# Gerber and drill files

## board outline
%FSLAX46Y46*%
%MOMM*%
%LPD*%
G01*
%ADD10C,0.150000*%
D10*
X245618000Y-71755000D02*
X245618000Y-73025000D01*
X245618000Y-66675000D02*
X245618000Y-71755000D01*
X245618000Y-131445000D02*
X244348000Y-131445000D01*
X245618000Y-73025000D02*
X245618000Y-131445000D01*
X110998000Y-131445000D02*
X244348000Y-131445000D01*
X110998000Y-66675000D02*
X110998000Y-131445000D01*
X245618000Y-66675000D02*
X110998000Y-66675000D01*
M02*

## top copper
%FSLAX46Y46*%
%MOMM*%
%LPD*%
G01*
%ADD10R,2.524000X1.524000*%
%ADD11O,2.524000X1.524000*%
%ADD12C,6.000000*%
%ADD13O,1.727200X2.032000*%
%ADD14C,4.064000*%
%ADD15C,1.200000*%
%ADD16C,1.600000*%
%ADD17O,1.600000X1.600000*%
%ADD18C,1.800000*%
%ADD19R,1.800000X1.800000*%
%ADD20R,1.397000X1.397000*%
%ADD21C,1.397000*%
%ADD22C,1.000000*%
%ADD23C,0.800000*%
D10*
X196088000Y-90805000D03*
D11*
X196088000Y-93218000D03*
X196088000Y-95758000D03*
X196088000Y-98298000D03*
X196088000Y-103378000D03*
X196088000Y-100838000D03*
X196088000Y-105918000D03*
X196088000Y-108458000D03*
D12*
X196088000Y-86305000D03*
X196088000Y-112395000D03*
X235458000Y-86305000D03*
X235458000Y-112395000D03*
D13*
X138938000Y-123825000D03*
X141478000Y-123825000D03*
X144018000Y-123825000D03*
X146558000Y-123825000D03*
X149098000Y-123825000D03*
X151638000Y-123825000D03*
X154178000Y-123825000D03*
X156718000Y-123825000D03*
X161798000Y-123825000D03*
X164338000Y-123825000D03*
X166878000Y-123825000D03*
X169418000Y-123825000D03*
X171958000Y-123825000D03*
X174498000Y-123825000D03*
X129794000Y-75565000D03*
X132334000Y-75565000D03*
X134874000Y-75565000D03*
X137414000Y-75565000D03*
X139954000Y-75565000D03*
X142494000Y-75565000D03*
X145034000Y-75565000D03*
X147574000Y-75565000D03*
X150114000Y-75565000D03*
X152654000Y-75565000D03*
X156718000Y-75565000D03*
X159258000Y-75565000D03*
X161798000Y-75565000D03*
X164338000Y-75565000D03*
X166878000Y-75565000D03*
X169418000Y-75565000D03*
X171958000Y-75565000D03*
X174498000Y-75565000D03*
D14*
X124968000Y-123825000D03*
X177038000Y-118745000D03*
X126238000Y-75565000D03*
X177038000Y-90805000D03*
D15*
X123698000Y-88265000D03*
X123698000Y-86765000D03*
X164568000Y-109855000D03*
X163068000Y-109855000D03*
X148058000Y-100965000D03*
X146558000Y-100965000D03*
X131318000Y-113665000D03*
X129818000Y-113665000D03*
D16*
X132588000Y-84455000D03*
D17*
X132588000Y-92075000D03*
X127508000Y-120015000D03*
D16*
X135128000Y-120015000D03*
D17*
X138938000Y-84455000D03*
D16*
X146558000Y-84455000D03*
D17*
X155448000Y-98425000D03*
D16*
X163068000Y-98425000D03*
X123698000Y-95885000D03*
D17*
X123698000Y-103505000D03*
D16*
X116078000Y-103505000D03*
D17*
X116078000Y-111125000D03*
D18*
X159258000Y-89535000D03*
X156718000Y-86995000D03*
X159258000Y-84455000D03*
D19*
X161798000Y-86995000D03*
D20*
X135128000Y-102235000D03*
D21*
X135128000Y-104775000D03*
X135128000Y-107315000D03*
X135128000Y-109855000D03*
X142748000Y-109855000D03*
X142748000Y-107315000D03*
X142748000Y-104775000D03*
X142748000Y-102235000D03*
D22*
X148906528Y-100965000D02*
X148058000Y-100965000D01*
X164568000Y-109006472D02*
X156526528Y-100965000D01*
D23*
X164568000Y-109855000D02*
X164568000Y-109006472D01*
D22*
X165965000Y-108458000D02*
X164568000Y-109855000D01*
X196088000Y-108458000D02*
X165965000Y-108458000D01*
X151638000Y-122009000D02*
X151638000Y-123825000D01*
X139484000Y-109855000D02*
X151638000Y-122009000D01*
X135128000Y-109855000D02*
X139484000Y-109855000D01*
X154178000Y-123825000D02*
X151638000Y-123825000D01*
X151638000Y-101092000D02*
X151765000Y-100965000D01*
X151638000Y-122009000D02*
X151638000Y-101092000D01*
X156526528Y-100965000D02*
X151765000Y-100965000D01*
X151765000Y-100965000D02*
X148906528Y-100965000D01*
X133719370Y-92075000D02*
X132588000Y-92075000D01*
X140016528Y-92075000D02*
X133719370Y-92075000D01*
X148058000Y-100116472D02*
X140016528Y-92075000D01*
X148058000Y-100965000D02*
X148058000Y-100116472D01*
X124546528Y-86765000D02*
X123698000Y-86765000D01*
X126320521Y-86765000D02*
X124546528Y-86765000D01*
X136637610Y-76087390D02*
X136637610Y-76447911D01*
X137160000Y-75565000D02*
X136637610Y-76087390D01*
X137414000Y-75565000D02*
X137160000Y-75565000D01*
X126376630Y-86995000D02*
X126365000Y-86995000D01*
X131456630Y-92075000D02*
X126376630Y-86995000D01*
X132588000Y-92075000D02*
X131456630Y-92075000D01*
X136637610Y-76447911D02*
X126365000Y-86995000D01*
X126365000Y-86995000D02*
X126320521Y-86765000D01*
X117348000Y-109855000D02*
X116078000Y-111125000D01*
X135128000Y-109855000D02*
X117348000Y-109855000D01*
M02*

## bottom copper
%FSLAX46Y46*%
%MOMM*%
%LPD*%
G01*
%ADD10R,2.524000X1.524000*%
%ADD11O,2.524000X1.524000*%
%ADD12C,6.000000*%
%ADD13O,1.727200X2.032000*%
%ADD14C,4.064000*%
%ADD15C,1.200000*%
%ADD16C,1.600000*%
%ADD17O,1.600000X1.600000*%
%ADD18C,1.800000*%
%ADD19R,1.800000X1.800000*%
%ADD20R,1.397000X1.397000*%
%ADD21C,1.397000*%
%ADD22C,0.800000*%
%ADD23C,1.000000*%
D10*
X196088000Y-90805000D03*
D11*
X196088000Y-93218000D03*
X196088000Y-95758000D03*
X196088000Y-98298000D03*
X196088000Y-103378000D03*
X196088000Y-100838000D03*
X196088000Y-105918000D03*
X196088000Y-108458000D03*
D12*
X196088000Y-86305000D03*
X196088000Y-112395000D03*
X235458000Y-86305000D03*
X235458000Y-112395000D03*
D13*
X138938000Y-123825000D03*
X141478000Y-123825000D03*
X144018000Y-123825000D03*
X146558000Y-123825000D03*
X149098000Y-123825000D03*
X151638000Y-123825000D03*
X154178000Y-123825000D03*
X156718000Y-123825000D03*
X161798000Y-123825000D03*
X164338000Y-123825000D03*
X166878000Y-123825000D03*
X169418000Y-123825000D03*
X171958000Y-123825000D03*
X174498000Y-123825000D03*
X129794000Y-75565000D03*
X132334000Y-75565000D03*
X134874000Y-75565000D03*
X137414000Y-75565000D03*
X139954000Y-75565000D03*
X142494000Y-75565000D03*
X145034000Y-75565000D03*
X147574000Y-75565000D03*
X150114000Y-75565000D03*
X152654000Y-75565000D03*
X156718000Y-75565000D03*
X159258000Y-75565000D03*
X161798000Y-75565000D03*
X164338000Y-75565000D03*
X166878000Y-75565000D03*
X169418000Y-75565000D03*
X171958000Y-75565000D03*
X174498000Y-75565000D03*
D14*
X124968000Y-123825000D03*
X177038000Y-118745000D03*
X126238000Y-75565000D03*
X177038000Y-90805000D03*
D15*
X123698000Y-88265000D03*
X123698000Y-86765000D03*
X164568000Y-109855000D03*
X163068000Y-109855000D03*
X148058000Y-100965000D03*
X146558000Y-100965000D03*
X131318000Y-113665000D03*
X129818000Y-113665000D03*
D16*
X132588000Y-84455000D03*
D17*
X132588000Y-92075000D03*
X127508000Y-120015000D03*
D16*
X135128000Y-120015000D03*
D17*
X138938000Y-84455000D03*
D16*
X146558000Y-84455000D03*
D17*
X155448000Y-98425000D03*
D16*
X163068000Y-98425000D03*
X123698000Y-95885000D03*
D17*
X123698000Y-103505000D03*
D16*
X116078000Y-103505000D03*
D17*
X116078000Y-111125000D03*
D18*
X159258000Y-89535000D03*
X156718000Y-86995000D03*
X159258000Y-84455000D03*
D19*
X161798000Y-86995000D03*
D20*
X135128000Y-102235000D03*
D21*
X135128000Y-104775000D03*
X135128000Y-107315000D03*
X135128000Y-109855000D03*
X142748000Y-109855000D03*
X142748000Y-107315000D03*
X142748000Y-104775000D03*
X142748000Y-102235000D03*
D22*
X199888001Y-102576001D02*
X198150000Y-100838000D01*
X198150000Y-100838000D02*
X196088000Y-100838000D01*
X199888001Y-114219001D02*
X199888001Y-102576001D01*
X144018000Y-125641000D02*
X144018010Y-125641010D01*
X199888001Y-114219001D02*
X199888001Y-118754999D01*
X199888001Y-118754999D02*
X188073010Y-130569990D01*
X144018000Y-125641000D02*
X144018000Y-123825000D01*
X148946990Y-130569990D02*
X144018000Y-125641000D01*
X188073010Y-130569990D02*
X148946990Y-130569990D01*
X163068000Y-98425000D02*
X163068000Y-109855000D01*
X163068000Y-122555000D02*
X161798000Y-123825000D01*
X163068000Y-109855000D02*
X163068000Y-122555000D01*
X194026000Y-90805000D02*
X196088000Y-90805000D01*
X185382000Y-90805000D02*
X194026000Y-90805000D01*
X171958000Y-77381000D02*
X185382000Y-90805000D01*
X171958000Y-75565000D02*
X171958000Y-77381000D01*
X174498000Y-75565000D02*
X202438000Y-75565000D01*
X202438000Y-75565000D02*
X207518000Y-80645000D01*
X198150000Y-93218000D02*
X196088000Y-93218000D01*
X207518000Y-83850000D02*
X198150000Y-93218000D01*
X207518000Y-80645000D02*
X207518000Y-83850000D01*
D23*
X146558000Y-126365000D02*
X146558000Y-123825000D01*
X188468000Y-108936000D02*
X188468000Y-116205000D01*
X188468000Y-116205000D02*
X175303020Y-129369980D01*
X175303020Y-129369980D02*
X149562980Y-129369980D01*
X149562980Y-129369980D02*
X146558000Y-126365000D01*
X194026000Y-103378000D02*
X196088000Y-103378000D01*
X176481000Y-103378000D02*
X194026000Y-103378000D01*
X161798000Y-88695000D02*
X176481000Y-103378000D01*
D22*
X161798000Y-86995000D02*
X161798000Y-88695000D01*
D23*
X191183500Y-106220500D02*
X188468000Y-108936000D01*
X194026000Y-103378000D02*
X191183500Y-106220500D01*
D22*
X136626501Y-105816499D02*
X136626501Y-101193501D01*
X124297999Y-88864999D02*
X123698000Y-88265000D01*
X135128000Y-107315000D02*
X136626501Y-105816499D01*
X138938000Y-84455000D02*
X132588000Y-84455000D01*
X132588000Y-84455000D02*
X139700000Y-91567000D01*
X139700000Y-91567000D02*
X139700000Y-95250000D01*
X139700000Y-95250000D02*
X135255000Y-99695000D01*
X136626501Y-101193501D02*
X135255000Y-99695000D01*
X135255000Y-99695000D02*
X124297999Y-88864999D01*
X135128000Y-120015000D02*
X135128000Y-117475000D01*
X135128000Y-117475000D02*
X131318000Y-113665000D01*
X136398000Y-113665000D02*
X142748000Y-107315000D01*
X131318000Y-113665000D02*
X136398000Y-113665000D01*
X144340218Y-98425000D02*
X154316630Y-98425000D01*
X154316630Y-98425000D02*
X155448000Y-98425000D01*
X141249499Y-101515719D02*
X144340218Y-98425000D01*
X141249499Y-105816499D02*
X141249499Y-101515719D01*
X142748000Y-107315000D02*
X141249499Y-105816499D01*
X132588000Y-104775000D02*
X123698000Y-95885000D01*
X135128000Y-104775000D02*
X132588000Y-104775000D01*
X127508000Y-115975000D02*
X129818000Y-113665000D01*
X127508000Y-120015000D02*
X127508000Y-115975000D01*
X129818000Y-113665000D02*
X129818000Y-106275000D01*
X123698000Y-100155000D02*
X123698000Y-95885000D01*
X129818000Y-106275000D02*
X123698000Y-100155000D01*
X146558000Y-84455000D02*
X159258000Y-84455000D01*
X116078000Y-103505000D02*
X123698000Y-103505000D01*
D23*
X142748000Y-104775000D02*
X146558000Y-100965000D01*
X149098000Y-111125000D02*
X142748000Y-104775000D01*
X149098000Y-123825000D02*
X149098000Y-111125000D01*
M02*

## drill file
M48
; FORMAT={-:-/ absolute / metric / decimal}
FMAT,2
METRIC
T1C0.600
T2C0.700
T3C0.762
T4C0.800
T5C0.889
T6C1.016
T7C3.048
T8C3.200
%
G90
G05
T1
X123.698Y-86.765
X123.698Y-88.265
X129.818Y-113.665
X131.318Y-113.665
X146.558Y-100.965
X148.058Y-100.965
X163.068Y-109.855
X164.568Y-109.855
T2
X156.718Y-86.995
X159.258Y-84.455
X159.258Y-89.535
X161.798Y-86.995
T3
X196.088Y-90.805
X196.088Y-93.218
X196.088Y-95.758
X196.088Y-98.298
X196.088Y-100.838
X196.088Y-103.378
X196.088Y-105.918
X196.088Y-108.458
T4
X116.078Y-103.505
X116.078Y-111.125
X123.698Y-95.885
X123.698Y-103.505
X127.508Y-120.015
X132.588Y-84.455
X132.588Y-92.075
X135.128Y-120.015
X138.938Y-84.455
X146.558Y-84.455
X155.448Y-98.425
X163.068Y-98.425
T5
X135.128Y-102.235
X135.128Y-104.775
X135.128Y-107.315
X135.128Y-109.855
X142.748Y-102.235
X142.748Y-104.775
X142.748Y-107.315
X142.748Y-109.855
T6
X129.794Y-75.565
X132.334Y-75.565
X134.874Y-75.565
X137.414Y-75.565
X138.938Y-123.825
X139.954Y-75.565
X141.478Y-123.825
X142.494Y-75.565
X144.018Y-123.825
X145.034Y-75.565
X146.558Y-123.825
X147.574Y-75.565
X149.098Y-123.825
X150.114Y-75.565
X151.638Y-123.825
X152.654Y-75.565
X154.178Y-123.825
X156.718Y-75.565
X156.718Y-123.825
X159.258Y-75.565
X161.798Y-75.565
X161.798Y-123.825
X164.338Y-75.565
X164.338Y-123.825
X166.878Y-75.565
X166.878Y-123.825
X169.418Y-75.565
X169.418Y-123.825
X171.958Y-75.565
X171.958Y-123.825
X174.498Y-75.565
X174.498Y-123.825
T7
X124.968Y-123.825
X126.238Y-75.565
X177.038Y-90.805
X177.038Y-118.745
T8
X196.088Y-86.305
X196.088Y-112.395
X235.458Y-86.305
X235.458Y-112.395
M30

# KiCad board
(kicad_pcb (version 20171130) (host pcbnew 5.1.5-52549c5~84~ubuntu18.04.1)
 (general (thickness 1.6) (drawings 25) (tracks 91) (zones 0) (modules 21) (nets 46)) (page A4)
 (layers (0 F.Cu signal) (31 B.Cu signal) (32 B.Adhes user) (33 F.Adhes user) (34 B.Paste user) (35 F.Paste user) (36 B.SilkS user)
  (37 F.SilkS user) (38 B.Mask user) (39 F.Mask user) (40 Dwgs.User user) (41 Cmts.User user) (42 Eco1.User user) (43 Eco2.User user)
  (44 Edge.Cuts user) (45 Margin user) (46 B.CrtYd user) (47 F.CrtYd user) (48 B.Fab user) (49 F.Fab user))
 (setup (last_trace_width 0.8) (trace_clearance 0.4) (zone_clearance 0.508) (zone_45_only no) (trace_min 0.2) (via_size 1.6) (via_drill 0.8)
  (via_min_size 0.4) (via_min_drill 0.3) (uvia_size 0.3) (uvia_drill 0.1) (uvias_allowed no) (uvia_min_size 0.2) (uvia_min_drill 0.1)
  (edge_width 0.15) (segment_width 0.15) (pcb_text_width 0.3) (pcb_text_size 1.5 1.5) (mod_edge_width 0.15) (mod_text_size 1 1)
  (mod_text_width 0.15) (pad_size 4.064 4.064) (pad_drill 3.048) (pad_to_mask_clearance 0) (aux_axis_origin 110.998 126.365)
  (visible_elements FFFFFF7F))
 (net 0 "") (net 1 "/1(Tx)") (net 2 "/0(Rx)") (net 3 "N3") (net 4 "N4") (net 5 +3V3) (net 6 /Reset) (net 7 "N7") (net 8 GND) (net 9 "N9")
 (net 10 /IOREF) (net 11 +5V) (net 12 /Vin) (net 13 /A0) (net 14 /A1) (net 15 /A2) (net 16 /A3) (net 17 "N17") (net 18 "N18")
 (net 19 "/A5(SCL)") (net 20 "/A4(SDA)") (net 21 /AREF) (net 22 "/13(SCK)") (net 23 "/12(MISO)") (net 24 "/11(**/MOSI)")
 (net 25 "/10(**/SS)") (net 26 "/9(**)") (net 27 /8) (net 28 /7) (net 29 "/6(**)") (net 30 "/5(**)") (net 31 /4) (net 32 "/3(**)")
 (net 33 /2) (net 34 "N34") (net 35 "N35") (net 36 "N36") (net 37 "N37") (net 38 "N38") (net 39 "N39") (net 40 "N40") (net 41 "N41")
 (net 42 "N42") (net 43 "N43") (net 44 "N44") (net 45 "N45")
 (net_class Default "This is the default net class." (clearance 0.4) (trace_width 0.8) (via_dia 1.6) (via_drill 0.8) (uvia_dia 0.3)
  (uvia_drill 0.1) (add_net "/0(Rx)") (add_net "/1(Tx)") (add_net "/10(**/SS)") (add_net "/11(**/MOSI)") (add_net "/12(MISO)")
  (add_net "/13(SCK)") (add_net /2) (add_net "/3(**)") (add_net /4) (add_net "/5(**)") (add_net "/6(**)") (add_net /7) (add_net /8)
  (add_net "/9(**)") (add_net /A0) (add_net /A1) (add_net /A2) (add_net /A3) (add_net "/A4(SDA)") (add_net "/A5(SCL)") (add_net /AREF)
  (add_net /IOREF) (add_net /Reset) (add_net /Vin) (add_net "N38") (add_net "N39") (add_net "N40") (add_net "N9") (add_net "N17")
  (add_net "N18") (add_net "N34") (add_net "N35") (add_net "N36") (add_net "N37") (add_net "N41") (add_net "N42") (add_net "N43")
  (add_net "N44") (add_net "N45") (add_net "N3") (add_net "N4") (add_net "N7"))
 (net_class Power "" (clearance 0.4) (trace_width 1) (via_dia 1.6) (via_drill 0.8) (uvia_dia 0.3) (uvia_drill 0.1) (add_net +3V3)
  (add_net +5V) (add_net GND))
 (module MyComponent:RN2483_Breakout (layer F.Cu) (at 196.088 90.805 270)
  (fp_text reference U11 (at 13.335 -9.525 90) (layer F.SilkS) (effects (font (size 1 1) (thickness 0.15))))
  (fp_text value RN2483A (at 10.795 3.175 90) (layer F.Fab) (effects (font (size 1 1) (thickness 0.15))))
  (pad 1 thru_hole rect (at 0 0 270) (size 1.524 2.524) (drill 0.762) (layers *.Cu *.Mask) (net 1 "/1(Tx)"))
  (pad 2 thru_hole oval (at 2.413 0 270) (size 1.524 2.524) (drill 0.762) (layers *.Cu *.Mask) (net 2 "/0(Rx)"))
  (pad 3 thru_hole oval (at 4.953 0 270) (size 1.524 2.524) (drill 0.762) (layers *.Cu *.Mask) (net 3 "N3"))
  (pad 4 thru_hole oval (at 7.493 0 270) (size 1.524 2.524) (drill 0.762) (layers *.Cu *.Mask) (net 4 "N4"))
  (pad 6 thru_hole oval (at 12.573 0 270) (size 1.524 2.524) (drill 0.762) (layers *.Cu *.Mask) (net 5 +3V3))
  (pad 5 thru_hole oval (at 10.033 0 270) (size 1.524 2.524) (drill 0.762) (layers *.Cu *.Mask) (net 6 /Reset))
  (pad 7 thru_hole oval (at 15.113 0 270) (size 1.524 2.524) (drill 0.762) (layers *.Cu *.Mask) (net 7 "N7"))
  (pad 8 thru_hole oval (at 17.653 0 270) (size 1.524 2.524) (drill 0.762) (layers *.Cu *.Mask) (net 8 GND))
  (pad "" np_thru_hole circle (at -4.5 0 270) (size 6 6) (drill 3.2) (layers *.Cu *.Mask))
  (pad "" np_thru_hole circle (at 21.59 0 270) (size 6 6) (drill 3.2) (layers *.Cu *.Mask))
  (pad "" np_thru_hole circle (at -4.5 -39.37 270) (size 6 6) (drill 3.2) (layers *.Cu *.Mask))
  (pad "" np_thru_hole circle (at 21.59 -39.37 270) (size 6 6) (drill 3.2) (layers *.Cu *.Mask)))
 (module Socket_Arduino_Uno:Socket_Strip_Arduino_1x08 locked (layer F.Cu) (at 138.938 123.825)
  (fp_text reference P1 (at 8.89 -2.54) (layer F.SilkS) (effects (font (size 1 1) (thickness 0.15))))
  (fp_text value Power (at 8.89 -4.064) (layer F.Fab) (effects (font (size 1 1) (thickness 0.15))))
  (pad 1 thru_hole oval (at 0 0) (size 1.7272 2.032) (drill 1.016) (layers *.Cu *.Mask F.SilkS) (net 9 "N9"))
  (pad 2 thru_hole oval (at 2.54 0) (size 1.7272 2.032) (drill 1.016) (layers *.Cu *.Mask F.SilkS) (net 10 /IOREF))
  (pad 3 thru_hole oval (at 5.08 0) (size 1.7272 2.032) (drill 1.016) (layers *.Cu *.Mask F.SilkS) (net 6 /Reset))
  (pad 4 thru_hole oval (at 7.62 0) (size 1.7272 2.032) (drill 1.016) (layers *.Cu *.Mask F.SilkS) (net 5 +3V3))
  (pad 5 thru_hole oval (at 10.16 0) (size 1.7272 2.032) (drill 1.016) (layers *.Cu *.Mask F.SilkS) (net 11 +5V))
  (pad 6 thru_hole oval (at 12.7 0) (size 1.7272 2.032) (drill 1.016) (layers *.Cu *.Mask F.SilkS) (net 8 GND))
  (pad 7 thru_hole oval (at 15.24 0) (size 1.7272 2.032) (drill 1.016) (layers *.Cu *.Mask F.SilkS) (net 8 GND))
  (pad 8 thru_hole oval (at 17.78 0) (size 1.7272 2.032) (drill 1.016) (layers *.Cu *.Mask F.SilkS) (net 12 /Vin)))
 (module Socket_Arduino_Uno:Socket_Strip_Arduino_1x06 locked (layer F.Cu) (at 161.798 123.825)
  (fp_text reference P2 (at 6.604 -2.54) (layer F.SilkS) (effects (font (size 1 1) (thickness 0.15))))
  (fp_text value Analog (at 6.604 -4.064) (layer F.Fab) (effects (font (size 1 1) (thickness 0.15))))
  (pad 1 thru_hole oval (at 0 0) (size 1.7272 2.032) (drill 1.016) (layers *.Cu *.Mask F.SilkS) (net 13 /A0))
  (pad 2 thru_hole oval (at 2.54 0) (size 1.7272 2.032) (drill 1.016) (layers *.Cu *.Mask F.SilkS) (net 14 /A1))
  (pad 3 thru_hole oval (at 5.08 0) (size 1.7272 2.032) (drill 1.016) (layers *.Cu *.Mask F.SilkS) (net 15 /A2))
  (pad 4 thru_hole oval (at 7.62 0) (size 1.7272 2.032) (drill 1.016) (layers *.Cu *.Mask F.SilkS) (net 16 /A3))
  (pad 5 thru_hole oval (at 10.16 0) (size 1.7272 2.032) (drill 1.016) (layers *.Cu *.Mask F.SilkS) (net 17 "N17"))
  (pad 6 thru_hole oval (at 12.7 0) (size 1.7272 2.032) (drill 1.016) (layers *.Cu *.Mask F.SilkS) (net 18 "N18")))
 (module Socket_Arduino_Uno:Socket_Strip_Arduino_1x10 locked (layer F.Cu) (at 129.794 75.565)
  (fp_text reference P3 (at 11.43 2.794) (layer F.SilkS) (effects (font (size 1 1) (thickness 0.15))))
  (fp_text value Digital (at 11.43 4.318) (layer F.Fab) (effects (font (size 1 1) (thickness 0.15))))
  (pad 1 thru_hole oval (at 0 0) (size 1.7272 2.032) (drill 1.016) (layers *.Cu *.Mask F.SilkS) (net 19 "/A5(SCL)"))
  (pad 2 thru_hole oval (at 2.54 0) (size 1.7272 2.032) (drill 1.016) (layers *.Cu *.Mask F.SilkS) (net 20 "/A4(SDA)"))
  (pad 3 thru_hole oval (at 5.08 0) (size 1.7272 2.032) (drill 1.016) (layers *.Cu *.Mask F.SilkS) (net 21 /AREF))
  (pad 4 thru_hole oval (at 7.62 0) (size 1.7272 2.032) (drill 1.016) (layers *.Cu *.Mask F.SilkS) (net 8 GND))
  (pad 5 thru_hole oval (at 10.16 0) (size 1.7272 2.032) (drill 1.016) (layers *.Cu *.Mask F.SilkS) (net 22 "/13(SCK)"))
  (pad 6 thru_hole oval (at 12.7 0) (size 1.7272 2.032) (drill 1.016) (layers *.Cu *.Mask F.SilkS) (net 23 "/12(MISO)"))
  (pad 7 thru_hole oval (at 15.24 0) (size 1.7272 2.032) (drill 1.016) (layers *.Cu *.Mask F.SilkS) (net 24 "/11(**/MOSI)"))
  (pad 8 thru_hole oval (at 17.78 0) (size 1.7272 2.032) (drill 1.016) (layers *.Cu *.Mask F.SilkS) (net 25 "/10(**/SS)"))
  (pad 9 thru_hole oval (at 20.32 0) (size 1.7272 2.032) (drill 1.016) (layers *.Cu *.Mask F.SilkS) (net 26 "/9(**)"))
  (pad 10 thru_hole oval (at 22.86 0) (size 1.7272 2.032) (drill 1.016) (layers *.Cu *.Mask F.SilkS) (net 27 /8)))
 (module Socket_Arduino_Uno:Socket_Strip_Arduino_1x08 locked (layer F.Cu) (at 156.718 75.565)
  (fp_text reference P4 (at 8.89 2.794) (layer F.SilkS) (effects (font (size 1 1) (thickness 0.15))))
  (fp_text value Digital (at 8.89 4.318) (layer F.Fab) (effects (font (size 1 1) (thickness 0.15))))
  (pad 1 thru_hole oval (at 0 0) (size 1.7272 2.032) (drill 1.016) (layers *.Cu *.Mask F.SilkS) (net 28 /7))
  (pad 2 thru_hole oval (at 2.54 0) (size 1.7272 2.032) (drill 1.016) (layers *.Cu *.Mask F.SilkS) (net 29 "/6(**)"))
  (pad 3 thru_hole oval (at 5.08 0) (size 1.7272 2.032) (drill 1.016) (layers *.Cu *.Mask F.SilkS) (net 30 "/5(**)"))
  (pad 4 thru_hole oval (at 7.62 0) (size 1.7272 2.032) (drill 1.016) (layers *.Cu *.Mask F.SilkS) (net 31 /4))
  (pad 5 thru_hole oval (at 10.16 0) (size 1.7272 2.032) (drill 1.016) (layers *.Cu *.Mask F.SilkS) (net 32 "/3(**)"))
  (pad 6 thru_hole oval (at 12.7 0) (size 1.7272 2.032) (drill 1.016) (layers *.Cu *.Mask F.SilkS) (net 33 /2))
  (pad 7 thru_hole oval (at 15.24 0) (size 1.7272 2.032) (drill 1.016) (layers *.Cu *.Mask F.SilkS) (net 1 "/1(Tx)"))
  (pad 8 thru_hole oval (at 17.78 0) (size 1.7272 2.032) (drill 1.016) (layers *.Cu *.Mask F.SilkS) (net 2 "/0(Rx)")))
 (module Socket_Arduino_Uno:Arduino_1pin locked (layer F.Cu) (at 124.968 123.825)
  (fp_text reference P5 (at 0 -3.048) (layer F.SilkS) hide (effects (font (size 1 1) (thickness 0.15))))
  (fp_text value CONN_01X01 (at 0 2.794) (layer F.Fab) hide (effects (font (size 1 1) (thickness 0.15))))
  (pad 1 thru_hole circle (at 0 0) (size 4.064 4.064) (drill 3.048) (layers *.Cu *.Mask F.SilkS) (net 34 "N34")))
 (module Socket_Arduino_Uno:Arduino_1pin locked (layer F.Cu) (at 177.038 118.745)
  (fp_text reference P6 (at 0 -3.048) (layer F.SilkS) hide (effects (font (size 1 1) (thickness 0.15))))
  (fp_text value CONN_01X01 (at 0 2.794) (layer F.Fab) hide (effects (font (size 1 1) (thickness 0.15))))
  (pad 1 thru_hole circle (at 0 0) (size 4.064 4.064) (drill 3.048) (layers *.Cu *.Mask F.SilkS) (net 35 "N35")))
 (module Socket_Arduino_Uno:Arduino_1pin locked (layer F.Cu) (at 126.238 75.565)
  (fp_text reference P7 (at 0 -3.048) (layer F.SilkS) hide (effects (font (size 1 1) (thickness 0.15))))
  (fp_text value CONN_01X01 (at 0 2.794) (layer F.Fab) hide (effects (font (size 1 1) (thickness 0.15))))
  (pad 1 thru_hole circle (at 0 0) (size 4.064 4.064) (drill 3.048) (layers *.Cu *.Mask F.SilkS) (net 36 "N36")))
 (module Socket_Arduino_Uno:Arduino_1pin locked (layer F.Cu) (at 177.038 90.805)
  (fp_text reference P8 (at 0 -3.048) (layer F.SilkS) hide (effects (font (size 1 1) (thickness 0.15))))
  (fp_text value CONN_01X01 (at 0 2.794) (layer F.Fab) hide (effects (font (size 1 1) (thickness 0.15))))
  (pad 1 thru_hole circle (at 0 0) (size 4.064 4.064) (drill 3.048) (layers *.Cu *.Mask F.SilkS) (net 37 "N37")))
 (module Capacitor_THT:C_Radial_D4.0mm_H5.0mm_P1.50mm (layer F.Cu) (at 123.698 88.265 90)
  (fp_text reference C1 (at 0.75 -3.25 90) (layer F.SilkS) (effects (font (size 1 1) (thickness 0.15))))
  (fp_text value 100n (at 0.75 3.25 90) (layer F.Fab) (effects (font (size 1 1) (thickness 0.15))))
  (pad 1 thru_hole circle (at 0 0 90) (size 1.2 1.2) (drill 0.6) (layers *.Cu *.Mask) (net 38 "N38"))
  (pad 2 thru_hole circle (at 1.5 0 90) (size 1.2 1.2) (drill 0.6) (layers *.Cu *.Mask) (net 8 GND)))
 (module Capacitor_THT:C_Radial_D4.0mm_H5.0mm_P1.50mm (layer F.Cu) (at 163.068 109.855)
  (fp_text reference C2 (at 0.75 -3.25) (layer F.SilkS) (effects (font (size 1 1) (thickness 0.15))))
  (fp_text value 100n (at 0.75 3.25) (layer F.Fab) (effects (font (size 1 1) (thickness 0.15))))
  (pad 2 thru_hole circle (at 1.5 0) (size 1.2 1.2) (drill 0.6) (layers *.Cu *.Mask) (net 8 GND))
  (pad 1 thru_hole circle (at 0 0) (size 1.2 1.2) (drill 0.6) (layers *.Cu *.Mask) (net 13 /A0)))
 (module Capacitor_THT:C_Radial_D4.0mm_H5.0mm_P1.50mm (layer F.Cu) (at 146.558 100.965)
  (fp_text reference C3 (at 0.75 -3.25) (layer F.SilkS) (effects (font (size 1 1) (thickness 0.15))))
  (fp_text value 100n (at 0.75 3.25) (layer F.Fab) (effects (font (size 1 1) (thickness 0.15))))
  (pad 2 thru_hole circle (at 1.5 0) (size 1.2 1.2) (drill 0.6) (layers *.Cu *.Mask) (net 8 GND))
  (pad 1 thru_hole circle (at 0 0) (size 1.2 1.2) (drill 0.6) (layers *.Cu *.Mask) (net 11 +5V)))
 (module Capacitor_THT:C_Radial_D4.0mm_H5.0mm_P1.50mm (layer F.Cu) (at 131.318 113.665 180)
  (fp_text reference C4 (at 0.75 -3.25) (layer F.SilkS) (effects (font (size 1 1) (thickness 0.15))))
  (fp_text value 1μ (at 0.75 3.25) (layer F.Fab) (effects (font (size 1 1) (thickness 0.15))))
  (pad 1 thru_hole circle (at 0 0 180) (size 1.2 1.2) (drill 0.6) (layers *.Cu *.Mask) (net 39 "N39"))
  (pad 2 thru_hole circle (at 1.5 0 180) (size 1.2 1.2) (drill 0.6) (layers *.Cu *.Mask) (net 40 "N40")))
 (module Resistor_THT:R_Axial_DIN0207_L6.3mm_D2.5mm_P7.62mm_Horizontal (layer F.Cu) (at 132.588 84.455 270)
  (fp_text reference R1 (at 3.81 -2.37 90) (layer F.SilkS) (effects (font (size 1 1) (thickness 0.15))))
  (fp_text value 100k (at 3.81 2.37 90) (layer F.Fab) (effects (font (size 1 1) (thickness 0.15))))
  (pad 1 thru_hole circle (at 0 0 270) (size 1.6 1.6) (drill 0.8) (layers *.Cu *.Mask) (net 38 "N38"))
  (pad 2 thru_hole oval (at 7.62 0 270) (size 1.6 1.6) (drill 0.8) (layers *.Cu *.Mask) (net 8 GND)))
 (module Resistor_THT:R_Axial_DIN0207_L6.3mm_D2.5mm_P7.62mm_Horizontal (layer F.Cu) (at 135.128 120.015 180)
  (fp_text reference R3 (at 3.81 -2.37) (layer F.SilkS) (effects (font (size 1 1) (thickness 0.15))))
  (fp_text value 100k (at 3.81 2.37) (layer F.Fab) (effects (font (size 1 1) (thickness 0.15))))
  (pad 2 thru_hole oval (at 7.62 0 180) (size 1.6 1.6) (drill 0.8) (layers *.Cu *.Mask) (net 40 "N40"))
  (pad 1 thru_hole circle (at 0 0 180) (size 1.6 1.6) (drill 0.8) (layers *.Cu *.Mask) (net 39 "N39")))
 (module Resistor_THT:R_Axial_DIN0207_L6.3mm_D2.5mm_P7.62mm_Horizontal (layer F.Cu) (at 146.558 84.455 180)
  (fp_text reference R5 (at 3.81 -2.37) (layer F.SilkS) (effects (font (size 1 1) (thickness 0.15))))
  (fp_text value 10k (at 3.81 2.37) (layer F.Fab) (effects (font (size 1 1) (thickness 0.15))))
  (pad 2 thru_hole oval (at 7.62 0 180) (size 1.6 1.6) (drill 0.8) (layers *.Cu *.Mask) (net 38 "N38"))
  (pad 1 thru_hole circle (at 0 0 180) (size 1.6 1.6) (drill 0.8) (layers *.Cu *.Mask) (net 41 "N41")))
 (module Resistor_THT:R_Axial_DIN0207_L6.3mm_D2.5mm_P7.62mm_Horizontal (layer F.Cu) (at 163.068 98.425 180)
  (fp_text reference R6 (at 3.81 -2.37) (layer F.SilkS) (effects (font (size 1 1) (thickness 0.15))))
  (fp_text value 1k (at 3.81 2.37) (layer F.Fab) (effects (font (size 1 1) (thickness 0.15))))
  (pad 2 thru_hole oval (at 7.62 0 180) (size 1.6 1.6) (drill 0.8) (layers *.Cu *.Mask) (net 39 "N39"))
  (pad 1 thru_hole circle (at 0 0 180) (size 1.6 1.6) (drill 0.8) (layers *.Cu *.Mask) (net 13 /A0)))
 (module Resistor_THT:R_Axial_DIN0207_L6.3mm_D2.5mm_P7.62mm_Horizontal (layer F.Cu) (at 123.698 95.885 270)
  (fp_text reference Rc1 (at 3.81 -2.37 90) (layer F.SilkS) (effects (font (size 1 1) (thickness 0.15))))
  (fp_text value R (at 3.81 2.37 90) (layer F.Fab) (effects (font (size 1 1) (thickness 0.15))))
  (pad 1 thru_hole circle (at 0 0 270) (size 1.6 1.6) (drill 0.8) (layers *.Cu *.Mask) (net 40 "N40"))
  (pad 2 thru_hole oval (at 7.62 0 270) (size 1.6 1.6) (drill 0.8) (layers *.Cu *.Mask) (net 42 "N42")))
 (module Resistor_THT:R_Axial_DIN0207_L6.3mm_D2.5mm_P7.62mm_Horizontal (layer F.Cu) (at 116.078 103.505 270)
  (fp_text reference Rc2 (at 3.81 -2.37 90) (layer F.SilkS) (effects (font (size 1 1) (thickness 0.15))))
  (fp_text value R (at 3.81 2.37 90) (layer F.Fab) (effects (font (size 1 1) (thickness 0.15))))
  (pad 1 thru_hole circle (at 0 0 270) (size 1.6 1.6) (drill 0.8) (layers *.Cu *.Mask) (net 42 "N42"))
  (pad 2 thru_hole oval (at 7.62 0 270) (size 1.6 1.6) (drill 0.8) (layers *.Cu *.Mask) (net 8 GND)))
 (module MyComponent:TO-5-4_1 (layer F.Cu) (at 161.798 86.995 180)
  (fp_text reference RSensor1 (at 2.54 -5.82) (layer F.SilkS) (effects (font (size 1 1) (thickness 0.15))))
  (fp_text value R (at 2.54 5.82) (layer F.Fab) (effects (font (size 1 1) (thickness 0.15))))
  (pad 4 thru_hole circle (at 2.54 -2.54 180) (size 1.8 1.8) (drill 0.7) (layers *.Cu *.Mask))
  (pad 3 thru_hole circle (at 5.08 0 180) (size 1.8 1.8) (drill 0.7) (layers *.Cu *.Mask))
  (pad 2 thru_hole circle (at 2.54 2.54 180) (size 1.8 1.8) (drill 0.7) (layers *.Cu *.Mask) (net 41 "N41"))
  (pad 1 thru_hole rect (at 0 0 180) (size 1.8 1.8) (drill 0.7) (layers *.Cu *.Mask) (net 5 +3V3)))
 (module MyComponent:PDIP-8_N (layer F.Cu) (at 142.748 109.855)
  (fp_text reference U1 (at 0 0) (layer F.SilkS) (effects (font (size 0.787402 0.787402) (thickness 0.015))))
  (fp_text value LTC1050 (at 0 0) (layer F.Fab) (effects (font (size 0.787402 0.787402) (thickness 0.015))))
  (pad 1 thru_hole rect (at -7.62 -7.62) (size 1.397 1.397) (drill 0.889) (layers *.Cu *.Mask) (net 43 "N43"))
  (pad 2 thru_hole circle (at -7.62 -5.08) (size 1.397 1.397) (drill 0.889) (layers *.Cu *.Mask) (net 40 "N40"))
  (pad 3 thru_hole circle (at -7.62 -2.54) (size 1.397 1.397) (drill 0.889) (layers *.Cu *.Mask) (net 38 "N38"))
  (pad 4 thru_hole circle (at -7.62 0) (size 1.397 1.397) (drill 0.889) (layers *.Cu *.Mask) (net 8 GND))
  (pad 5 thru_hole circle (at 0 0) (size 1.397 1.397) (drill 0.889) (layers *.Cu *.Mask) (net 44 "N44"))
  (pad 6 thru_hole circle (at 0 -2.54) (size 1.397 1.397) (drill 0.889) (layers *.Cu *.Mask) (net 39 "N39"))
  (pad 7 thru_hole circle (at 0 -5.08) (size 1.397 1.397) (drill 0.889) (layers *.Cu *.Mask) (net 11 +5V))
  (pad 8 thru_hole circle (at 0 -7.62) (size 1.397 1.397) (drill 0.889) (layers *.Cu *.Mask) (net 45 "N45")))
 (gr_line (start 245.618 71.755) (end 245.618 73.025) (layer Edge.Cuts) (width 0.15))
 (gr_line (start 245.618 66.675) (end 245.618 71.755) (layer Edge.Cuts) (width 0.15))
 (gr_line (start 245.618 131.445) (end 244.348 131.445) (layer Edge.Cuts) (width 0.15))
 (gr_line (start 245.618 73.025) (end 245.618 131.445) (layer Edge.Cuts) (width 0.15))
 (gr_line (start 110.998 131.445) (end 244.348 131.445) (angle 90) (layer Edge.Cuts) (width 0.15))
 (gr_line (start 110.998 66.675) (end 110.998 131.445) (angle 90) (layer Edge.Cuts) (width 0.15))
 (gr_line (start 245.618 66.675) (end 110.998 66.675) (angle 90) (layer Edge.Cuts) (width 0.15))
 (segment (start 199.888001 102.576001) (end 198.15 100.838) (width 0.8) (layer B.Cu) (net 6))
 (segment (start 198.15 100.838) (end 196.088 100.838) (width 0.8) (layer B.Cu) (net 6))
 (segment (start 199.888001 114.219001) (end 199.888001 102.576001) (width 0.8) (layer B.Cu) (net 6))
 (segment (start 144.018 125.641) (end 144.01801 125.64101) (width 0.8) (layer B.Cu) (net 6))
 (segment (start 199.888001 114.219001) (end 199.888001 118.754999) (width 0.8) (layer B.Cu) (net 6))
 (segment (start 199.888001 118.754999) (end 188.07301 130.56999) (width 0.8) (layer B.Cu) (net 6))
 (segment (start 144.018 125.641) (end 144.018 123.825) (width 0.8) (layer B.Cu) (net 6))
 (segment (start 148.94699 130.56999) (end 144.018 125.641) (width 0.8) (layer B.Cu) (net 6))
 (segment (start 188.07301 130.56999) (end 148.94699 130.56999) (width 0.8) (layer B.Cu) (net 6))
 (segment (start 163.068 98.425) (end 163.068 109.855) (width 0.8) (layer B.Cu) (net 13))
 (segment (start 163.068 122.555) (end 161.798 123.825) (width 0.8) (layer B.Cu) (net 13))
 (segment (start 163.068 109.855) (end 163.068 122.555) (width 0.8) (layer B.Cu) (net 13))
 (segment (start 194.026 90.805) (end 196.088 90.805) (width 0.8) (layer B.Cu) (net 1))
 (segment (start 185.382 90.805) (end 194.026 90.805) (width 0.8) (layer B.Cu) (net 1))
 (segment (start 171.958 77.381) (end 185.382 90.805) (width 0.8) (layer B.Cu) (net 1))
 (segment (start 171.958 75.565) (end 171.958 77.381) (width 0.8) (layer B.Cu) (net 1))
 (segment (start 174.498 75.565) (end 202.438 75.565) (width 0.8) (layer B.Cu) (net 2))
 (segment (start 202.438 75.565) (end 207.518 80.645) (width 0.8) (layer B.Cu) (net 2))
 (segment (start 198.15 93.218) (end 196.088 93.218) (width 0.8) (layer B.Cu) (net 2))
 (segment (start 207.518 83.85) (end 198.15 93.218) (width 0.8) (layer B.Cu) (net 2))
 (segment (start 207.518 80.645) (end 207.518 83.85) (width 0.8) (layer B.Cu) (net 2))
 (segment (start 146.558 126.365) (end 146.558 123.825) (width 1) (layer B.Cu) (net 5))
 (segment (start 188.468 108.936) (end 188.468 116.205) (width 1) (layer B.Cu) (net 5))
 (segment (start 188.468 116.205) (end 175.30302 129.36998) (width 1) (layer B.Cu) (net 5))
 (segment (start 175.30302 129.36998) (end 149.56298 129.36998) (width 1) (layer B.Cu) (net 5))
 (segment (start 149.56298 129.36998) (end 146.558 126.365) (width 1) (layer B.Cu) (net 5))
 (segment (start 194.026 103.378) (end 196.088 103.378) (width 1) (layer B.Cu) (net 5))
 (segment (start 176.481 103.378) (end 194.026 103.378) (width 1) (layer B.Cu) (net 5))
 (segment (start 161.798 88.695) (end 176.481 103.378) (width 1) (layer B.Cu) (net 5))
 (segment (start 161.798 86.995) (end 161.798 88.695) (width 0.8) (layer B.Cu) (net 5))
 (segment (start 191.1835 106.2205) (end 188.468 108.936) (width 1) (layer B.Cu) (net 5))
 (segment (start 194.026 103.378) (end 191.1835 106.2205) (width 1) (layer B.Cu) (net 5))
 (segment (start 136.626501 105.816499) (end 136.626501 101.193501) (width 0.8) (layer B.Cu) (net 38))
 (segment (start 124.297999 88.864999) (end 123.698 88.265) (width 0.8) (layer B.Cu) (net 38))
 (segment (start 135.128 107.315) (end 136.626501 105.816499) (width 0.8) (layer B.Cu) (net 38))
 (segment (start 138.938 84.455) (end 132.588 84.455) (width 0.8) (layer B.Cu) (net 38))
 (segment (start 132.588 84.455) (end 139.7 91.567) (width 0.8) (layer B.Cu) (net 38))
 (segment (start 139.7 91.567) (end 139.7 95.25) (width 0.8) (layer B.Cu) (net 38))
 (segment (start 139.7 95.25) (end 135.255 99.695) (width 0.8) (layer B.Cu) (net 38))
 (segment (start 136.626501 101.193501) (end 135.255 99.695) (width 0.8) (layer B.Cu) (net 38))
 (segment (start 135.255 99.695) (end 124.297999 88.864999) (width 0.8) (layer B.Cu) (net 38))
 (segment (start 135.128 120.015) (end 135.128 117.475) (width 0.8) (layer B.Cu) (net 39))
 (segment (start 135.128 117.475) (end 131.318 113.665) (width 0.8) (layer B.Cu) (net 39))
 (segment (start 136.398 113.665) (end 142.748 107.315) (width 0.8) (layer B.Cu) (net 39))
 (segment (start 131.318 113.665) (end 136.398 113.665) (width 0.8) (layer B.Cu) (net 39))
 (segment (start 144.340218 98.425) (end 154.31663 98.425) (width 0.8) (layer B.Cu) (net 39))
 (segment (start 154.31663 98.425) (end 155.448 98.425) (width 0.8) (layer B.Cu) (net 39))
 (segment (start 141.249499 101.515719) (end 144.340218 98.425) (width 0.8) (layer B.Cu) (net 39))
 (segment (start 141.249499 105.816499) (end 141.249499 101.515719) (width 0.8) (layer B.Cu) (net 39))
 (segment (start 142.748 107.315) (end 141.249499 105.816499) (width 0.8) (layer B.Cu) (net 39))
 (segment (start 132.588 104.775) (end 123.698 95.885) (width 0.8) (layer B.Cu) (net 40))
 (segment (start 135.128 104.775) (end 132.588 104.775) (width 0.8) (layer B.Cu) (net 40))
 (segment (start 127.508 115.975) (end 129.818 113.665) (width 0.8) (layer B.Cu) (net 40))
 (segment (start 127.508 120.015) (end 127.508 115.975) (width 0.8) (layer B.Cu) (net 40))
 (segment (start 129.818 113.665) (end 129.818 106.275) (width 0.8) (layer B.Cu) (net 40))
 (segment (start 123.698 100.155) (end 123.698 95.885) (width 0.8) (layer B.Cu) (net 40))
 (segment (start 129.818 106.275) (end 123.698 100.155) (width 0.8) (layer B.Cu) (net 40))
 (segment (start 146.558 84.455) (end 159.258 84.455) (width 0.8) (layer B.Cu) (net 41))
 (segment (start 116.078 103.505) (end 123.698 103.505) (width 0.8) (layer B.Cu) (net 42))
 (segment (start 148.906528 100.965) (end 148.058 100.965) (width 1) (layer F.Cu) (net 8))
 (segment (start 164.568 109.006472) (end 156.526528 100.965) (width 1) (layer F.Cu) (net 8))
 (segment (start 164.568 109.855) (end 164.568 109.006472) (width 0.8) (layer F.Cu) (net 8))
 (segment (start 165.965 108.458) (end 164.568 109.855) (width 1) (layer F.Cu) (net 8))
 (segment (start 196.088 108.458) (end 165.965 108.458) (width 1) (layer F.Cu) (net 8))
 (segment (start 151.638 122.009) (end 151.638 123.825) (width 1) (layer F.Cu) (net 8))
 (segment (start 139.484 109.855) (end 151.638 122.009) (width 1) (layer F.Cu) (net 8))
 (segment (start 135.128 109.855) (end 139.484 109.855) (width 1) (layer F.Cu) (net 8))
 (segment (start 154.178 123.825) (end 151.638 123.825) (width 1) (layer F.Cu) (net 8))
 (segment (start 151.638 101.092) (end 151.765 100.965) (width 1) (layer F.Cu) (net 8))
 (segment (start 151.638 122.009) (end 151.638 101.092) (width 1) (layer F.Cu) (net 8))
 (segment (start 156.526528 100.965) (end 151.765 100.965) (width 1) (layer F.Cu) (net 8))
 (segment (start 151.765 100.965) (end 148.906528 100.965) (width 1) (layer F.Cu) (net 8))
 (segment (start 133.71937 92.075) (end 132.588 92.075) (width 1) (layer F.Cu) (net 8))
 (segment (start 140.016528 92.075) (end 133.71937 92.075) (width 1) (layer F.Cu) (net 8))
 (segment (start 148.058 100.116472) (end 140.016528 92.075) (width 1) (layer F.Cu) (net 8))
 (segment (start 148.058 100.965) (end 148.058 100.116472) (width 1) (layer F.Cu) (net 8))
 (segment (start 124.546528 86.765) (end 123.698 86.765) (width 1) (layer F.Cu) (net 8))
 (segment (start 126.320521 86.765) (end 124.546528 86.765) (width 1) (layer F.Cu) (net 8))
 (segment (start 136.63761 76.08739) (end 136.63761 76.447911) (width 1) (layer F.Cu) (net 8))
 (segment (start 137.16 75.565) (end 136.63761 76.08739) (width 1) (layer F.Cu) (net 8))
 (segment (start 137.414 75.565) (end 137.16 75.565) (width 1) (layer F.Cu) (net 8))
 (segment (start 126.37663 86.995) (end 126.365 86.995) (width 1) (layer F.Cu) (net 8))
 (segment (start 131.45663 92.075) (end 126.37663 86.995) (width 1) (layer F.Cu) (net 8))
 (segment (start 132.588 92.075) (end 131.45663 92.075) (width 1) (layer F.Cu) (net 8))
 (segment (start 136.63761 76.447911) (end 126.365 86.995) (width 1) (layer F.Cu) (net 8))
 (segment (start 126.365 86.995) (end 126.320521 86.765) (width 1) (layer F.Cu) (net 8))
 (segment (start 117.348 109.855) (end 116.078 111.125) (width 1) (layer F.Cu) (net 8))
 (segment (start 135.128 109.855) (end 117.348 109.855) (width 1) (layer F.Cu) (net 8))
 (segment (start 142.748 104.775) (end 146.558 100.965) (width 1) (layer B.Cu) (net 11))
 (segment (start 149.098 111.125) (end 142.748 104.775) (width 1) (layer B.Cu) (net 11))
 (segment (start 149.098 123.825) (end 149.098 111.125) (width 1) (layer B.Cu) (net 11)))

